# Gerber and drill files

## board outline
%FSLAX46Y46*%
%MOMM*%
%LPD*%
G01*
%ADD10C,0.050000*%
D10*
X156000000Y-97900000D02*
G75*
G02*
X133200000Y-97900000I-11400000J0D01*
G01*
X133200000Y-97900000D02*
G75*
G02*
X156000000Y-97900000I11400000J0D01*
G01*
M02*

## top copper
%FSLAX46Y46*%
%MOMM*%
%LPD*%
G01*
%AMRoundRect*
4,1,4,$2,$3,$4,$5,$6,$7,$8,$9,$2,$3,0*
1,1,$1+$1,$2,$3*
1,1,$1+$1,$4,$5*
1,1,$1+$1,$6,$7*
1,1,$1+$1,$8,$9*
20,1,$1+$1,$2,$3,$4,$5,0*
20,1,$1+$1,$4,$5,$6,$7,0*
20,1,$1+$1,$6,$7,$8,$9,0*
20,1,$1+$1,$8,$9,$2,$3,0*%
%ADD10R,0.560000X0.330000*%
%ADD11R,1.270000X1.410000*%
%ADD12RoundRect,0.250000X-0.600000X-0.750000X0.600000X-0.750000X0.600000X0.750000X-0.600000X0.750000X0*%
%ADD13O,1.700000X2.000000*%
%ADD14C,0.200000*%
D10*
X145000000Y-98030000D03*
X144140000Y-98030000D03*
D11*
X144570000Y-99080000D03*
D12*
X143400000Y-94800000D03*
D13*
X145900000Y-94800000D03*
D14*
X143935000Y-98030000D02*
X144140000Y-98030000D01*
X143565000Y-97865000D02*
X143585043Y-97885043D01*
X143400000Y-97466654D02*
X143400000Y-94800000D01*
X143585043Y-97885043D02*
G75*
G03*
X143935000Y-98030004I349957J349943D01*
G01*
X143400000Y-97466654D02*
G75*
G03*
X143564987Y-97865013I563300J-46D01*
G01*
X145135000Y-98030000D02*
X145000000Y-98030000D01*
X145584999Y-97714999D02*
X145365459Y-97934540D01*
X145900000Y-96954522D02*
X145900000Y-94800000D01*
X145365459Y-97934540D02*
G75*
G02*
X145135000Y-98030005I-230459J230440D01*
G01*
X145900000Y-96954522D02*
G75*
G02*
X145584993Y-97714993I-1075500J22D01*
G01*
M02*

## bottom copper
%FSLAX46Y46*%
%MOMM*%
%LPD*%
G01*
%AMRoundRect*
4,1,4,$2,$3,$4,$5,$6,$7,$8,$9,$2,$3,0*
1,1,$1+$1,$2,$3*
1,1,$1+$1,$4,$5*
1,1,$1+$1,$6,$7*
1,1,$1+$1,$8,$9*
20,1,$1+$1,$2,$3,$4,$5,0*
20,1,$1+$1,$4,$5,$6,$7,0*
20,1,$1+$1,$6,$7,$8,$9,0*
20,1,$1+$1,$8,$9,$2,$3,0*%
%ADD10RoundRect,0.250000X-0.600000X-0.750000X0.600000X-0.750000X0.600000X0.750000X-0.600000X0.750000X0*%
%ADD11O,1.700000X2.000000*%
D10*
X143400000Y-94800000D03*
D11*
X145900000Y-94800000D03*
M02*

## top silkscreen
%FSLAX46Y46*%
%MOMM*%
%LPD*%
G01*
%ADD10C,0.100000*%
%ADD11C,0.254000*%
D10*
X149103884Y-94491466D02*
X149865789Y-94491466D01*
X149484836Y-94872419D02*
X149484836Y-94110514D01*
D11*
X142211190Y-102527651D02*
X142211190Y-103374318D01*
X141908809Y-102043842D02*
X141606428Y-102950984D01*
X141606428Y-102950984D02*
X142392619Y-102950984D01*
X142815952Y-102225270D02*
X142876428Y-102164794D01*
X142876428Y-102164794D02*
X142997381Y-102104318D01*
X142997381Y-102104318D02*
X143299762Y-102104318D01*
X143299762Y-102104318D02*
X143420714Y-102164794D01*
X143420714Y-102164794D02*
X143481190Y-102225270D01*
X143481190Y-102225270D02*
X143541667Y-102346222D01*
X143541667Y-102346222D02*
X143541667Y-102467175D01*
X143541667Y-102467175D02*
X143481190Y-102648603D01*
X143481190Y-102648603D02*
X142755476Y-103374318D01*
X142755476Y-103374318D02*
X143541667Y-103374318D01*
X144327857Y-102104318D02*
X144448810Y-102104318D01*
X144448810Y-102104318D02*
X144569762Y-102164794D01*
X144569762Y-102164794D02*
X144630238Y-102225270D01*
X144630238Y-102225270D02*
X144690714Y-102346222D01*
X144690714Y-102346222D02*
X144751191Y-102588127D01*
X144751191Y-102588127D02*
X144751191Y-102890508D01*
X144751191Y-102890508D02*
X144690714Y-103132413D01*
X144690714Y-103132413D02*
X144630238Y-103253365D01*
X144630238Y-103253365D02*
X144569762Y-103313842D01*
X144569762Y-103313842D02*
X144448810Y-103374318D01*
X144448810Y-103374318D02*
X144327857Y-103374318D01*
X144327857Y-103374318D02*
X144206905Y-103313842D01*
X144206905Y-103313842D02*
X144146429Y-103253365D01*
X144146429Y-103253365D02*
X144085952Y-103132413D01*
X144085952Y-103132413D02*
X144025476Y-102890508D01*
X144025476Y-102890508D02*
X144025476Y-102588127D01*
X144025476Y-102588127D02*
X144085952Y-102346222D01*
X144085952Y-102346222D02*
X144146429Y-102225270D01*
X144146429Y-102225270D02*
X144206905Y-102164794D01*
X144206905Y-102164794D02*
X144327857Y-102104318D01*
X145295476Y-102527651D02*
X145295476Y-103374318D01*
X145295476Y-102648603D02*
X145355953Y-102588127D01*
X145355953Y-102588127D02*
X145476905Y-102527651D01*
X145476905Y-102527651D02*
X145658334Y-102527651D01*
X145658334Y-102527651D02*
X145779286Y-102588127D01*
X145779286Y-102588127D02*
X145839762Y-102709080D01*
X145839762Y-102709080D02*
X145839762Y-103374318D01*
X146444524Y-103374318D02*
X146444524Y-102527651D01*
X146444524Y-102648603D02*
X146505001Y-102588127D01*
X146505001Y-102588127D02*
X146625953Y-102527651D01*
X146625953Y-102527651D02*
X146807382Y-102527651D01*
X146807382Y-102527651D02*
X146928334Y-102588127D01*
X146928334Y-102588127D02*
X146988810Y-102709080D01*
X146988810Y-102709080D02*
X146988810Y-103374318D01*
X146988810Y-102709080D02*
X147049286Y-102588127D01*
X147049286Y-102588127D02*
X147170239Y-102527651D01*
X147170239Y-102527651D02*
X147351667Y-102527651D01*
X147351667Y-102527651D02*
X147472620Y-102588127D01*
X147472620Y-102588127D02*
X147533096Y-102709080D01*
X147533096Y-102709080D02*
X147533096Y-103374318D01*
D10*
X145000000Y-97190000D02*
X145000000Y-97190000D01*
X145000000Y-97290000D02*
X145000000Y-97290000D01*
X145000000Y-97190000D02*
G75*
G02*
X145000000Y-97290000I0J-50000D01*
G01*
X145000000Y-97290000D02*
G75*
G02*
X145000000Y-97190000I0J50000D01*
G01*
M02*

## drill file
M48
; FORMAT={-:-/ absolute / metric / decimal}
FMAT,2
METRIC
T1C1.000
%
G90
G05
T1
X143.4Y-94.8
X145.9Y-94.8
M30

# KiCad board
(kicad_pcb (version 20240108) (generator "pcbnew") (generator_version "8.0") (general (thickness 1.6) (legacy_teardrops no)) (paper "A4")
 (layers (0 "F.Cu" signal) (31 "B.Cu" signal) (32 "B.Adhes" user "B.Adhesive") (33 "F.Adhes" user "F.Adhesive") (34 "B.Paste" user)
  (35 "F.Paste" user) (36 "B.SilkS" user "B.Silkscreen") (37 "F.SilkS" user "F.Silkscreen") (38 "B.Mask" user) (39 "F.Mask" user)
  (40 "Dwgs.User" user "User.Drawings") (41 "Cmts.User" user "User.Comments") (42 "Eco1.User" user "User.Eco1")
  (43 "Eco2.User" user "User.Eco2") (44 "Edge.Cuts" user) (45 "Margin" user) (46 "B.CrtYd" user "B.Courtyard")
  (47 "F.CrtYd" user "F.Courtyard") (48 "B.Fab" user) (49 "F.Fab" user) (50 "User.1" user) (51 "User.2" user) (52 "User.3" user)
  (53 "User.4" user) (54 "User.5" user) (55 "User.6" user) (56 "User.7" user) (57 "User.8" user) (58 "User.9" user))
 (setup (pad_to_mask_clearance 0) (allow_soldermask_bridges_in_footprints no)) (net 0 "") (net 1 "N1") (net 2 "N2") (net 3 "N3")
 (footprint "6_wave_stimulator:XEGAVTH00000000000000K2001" (layer "F.Cu") (at 144.57 98.79)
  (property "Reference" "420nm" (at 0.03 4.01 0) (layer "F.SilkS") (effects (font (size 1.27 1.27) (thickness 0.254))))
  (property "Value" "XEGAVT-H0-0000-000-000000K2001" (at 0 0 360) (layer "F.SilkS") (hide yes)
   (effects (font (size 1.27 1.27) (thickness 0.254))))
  (fp_line (start 0.43 -1.6) (end 0.43 -1.6) (stroke (width 0.1) (type solid)) (layer "F.SilkS"))
  (fp_line (start 0.43 -1.5) (end 0.43 -1.5) (stroke (width 0.1) (type solid)) (layer "F.SilkS"))
  (fp_arc (start 0.43 -1.6) (mid 0.48 -1.55) (end 0.43 -1.5) (stroke (width 0.1) (type solid)) (layer "F.SilkS"))
  (fp_arc (start 0.43 -1.5) (mid 0.38 -1.55) (end 0.43 -1.6) (stroke (width 0.1) (type solid)) (layer "F.SilkS"))
  (pad "1" smd rect (at 0.43 -0.76 90) (size 0.33 0.56) (layers "F.Cu" "F.Paste" "F.Mask") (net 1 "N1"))
  (pad "2" smd rect (at -0.43 -0.76 90) (size 0.33 0.56) (layers "F.Cu" "F.Paste" "F.Mask") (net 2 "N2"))
  (pad "3" smd rect (at 0 0.29 180) (size 1.27 1.41) (layers "F.Cu" "F.Paste" "F.Mask") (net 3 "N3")))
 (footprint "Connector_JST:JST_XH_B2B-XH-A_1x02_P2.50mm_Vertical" (layer "B.Cu") (at 143.4 94.8)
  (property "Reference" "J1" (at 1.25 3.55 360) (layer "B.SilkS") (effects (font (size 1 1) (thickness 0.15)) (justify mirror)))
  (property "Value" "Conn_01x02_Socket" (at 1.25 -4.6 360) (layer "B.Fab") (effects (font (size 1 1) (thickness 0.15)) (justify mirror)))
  (pad "1" thru_hole roundrect (at 0 0) (size 1.7 2) (drill 1) (layers "*.Cu" "*.Mask") (remove_unused_layers no)
   (roundrect_rratio 0.147059) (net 2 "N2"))
  (pad "2" thru_hole oval (at 2.5 0) (size 1.7 2) (drill 1) (layers "*.Cu" "*.Mask") (remove_unused_layers no) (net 1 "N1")))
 (gr_circle (center 144.6 97.9) (end 156 97.9) (stroke (width 0.05) (type default)) (fill none) (layer "Edge.Cuts"))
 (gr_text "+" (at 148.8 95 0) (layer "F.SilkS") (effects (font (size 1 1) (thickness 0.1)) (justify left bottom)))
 (segment (start 143.935 98.03) (end 144.14 98.03) (width 0.2) (layer "F.Cu") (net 2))
 (segment (start 143.565 97.865) (end 143.585043 97.885043) (width 0.2) (layer "F.Cu") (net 2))
 (segment (start 143.4 97.466654) (end 143.4 94.8) (width 0.2) (layer "F.Cu") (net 2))
 (arc (start 143.585043 97.885043) (mid 143.745604 97.992326) (end 143.935 98.03) (width 0.2) (layer "F.Cu") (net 2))
 (arc (start 143.4 97.466654) (mid 143.442882 97.682237) (end 143.565 97.865) (width 0.2) (layer "F.Cu") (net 2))
 (segment (start 145.135 98.03) (end 145 98.03) (width 0.2) (layer "F.Cu") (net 1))
 (segment (start 145.584999 97.714999) (end 145.365459 97.93454) (width 0.2) (layer "F.Cu") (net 1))
 (segment (start 145.9 96.954522) (end 145.9 94.8) (width 0.2) (layer "F.Cu") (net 1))
 (arc (start 145.365459 97.93454) (mid 145.259723 98.00519) (end 145.135 98.03) (width 0.2) (layer "F.Cu") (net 1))
 (arc (start 145.9 96.954522) (mid 145.818133 97.366089) (end 145.584999 97.714999) (width 0.2) (layer "F.Cu") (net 1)))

